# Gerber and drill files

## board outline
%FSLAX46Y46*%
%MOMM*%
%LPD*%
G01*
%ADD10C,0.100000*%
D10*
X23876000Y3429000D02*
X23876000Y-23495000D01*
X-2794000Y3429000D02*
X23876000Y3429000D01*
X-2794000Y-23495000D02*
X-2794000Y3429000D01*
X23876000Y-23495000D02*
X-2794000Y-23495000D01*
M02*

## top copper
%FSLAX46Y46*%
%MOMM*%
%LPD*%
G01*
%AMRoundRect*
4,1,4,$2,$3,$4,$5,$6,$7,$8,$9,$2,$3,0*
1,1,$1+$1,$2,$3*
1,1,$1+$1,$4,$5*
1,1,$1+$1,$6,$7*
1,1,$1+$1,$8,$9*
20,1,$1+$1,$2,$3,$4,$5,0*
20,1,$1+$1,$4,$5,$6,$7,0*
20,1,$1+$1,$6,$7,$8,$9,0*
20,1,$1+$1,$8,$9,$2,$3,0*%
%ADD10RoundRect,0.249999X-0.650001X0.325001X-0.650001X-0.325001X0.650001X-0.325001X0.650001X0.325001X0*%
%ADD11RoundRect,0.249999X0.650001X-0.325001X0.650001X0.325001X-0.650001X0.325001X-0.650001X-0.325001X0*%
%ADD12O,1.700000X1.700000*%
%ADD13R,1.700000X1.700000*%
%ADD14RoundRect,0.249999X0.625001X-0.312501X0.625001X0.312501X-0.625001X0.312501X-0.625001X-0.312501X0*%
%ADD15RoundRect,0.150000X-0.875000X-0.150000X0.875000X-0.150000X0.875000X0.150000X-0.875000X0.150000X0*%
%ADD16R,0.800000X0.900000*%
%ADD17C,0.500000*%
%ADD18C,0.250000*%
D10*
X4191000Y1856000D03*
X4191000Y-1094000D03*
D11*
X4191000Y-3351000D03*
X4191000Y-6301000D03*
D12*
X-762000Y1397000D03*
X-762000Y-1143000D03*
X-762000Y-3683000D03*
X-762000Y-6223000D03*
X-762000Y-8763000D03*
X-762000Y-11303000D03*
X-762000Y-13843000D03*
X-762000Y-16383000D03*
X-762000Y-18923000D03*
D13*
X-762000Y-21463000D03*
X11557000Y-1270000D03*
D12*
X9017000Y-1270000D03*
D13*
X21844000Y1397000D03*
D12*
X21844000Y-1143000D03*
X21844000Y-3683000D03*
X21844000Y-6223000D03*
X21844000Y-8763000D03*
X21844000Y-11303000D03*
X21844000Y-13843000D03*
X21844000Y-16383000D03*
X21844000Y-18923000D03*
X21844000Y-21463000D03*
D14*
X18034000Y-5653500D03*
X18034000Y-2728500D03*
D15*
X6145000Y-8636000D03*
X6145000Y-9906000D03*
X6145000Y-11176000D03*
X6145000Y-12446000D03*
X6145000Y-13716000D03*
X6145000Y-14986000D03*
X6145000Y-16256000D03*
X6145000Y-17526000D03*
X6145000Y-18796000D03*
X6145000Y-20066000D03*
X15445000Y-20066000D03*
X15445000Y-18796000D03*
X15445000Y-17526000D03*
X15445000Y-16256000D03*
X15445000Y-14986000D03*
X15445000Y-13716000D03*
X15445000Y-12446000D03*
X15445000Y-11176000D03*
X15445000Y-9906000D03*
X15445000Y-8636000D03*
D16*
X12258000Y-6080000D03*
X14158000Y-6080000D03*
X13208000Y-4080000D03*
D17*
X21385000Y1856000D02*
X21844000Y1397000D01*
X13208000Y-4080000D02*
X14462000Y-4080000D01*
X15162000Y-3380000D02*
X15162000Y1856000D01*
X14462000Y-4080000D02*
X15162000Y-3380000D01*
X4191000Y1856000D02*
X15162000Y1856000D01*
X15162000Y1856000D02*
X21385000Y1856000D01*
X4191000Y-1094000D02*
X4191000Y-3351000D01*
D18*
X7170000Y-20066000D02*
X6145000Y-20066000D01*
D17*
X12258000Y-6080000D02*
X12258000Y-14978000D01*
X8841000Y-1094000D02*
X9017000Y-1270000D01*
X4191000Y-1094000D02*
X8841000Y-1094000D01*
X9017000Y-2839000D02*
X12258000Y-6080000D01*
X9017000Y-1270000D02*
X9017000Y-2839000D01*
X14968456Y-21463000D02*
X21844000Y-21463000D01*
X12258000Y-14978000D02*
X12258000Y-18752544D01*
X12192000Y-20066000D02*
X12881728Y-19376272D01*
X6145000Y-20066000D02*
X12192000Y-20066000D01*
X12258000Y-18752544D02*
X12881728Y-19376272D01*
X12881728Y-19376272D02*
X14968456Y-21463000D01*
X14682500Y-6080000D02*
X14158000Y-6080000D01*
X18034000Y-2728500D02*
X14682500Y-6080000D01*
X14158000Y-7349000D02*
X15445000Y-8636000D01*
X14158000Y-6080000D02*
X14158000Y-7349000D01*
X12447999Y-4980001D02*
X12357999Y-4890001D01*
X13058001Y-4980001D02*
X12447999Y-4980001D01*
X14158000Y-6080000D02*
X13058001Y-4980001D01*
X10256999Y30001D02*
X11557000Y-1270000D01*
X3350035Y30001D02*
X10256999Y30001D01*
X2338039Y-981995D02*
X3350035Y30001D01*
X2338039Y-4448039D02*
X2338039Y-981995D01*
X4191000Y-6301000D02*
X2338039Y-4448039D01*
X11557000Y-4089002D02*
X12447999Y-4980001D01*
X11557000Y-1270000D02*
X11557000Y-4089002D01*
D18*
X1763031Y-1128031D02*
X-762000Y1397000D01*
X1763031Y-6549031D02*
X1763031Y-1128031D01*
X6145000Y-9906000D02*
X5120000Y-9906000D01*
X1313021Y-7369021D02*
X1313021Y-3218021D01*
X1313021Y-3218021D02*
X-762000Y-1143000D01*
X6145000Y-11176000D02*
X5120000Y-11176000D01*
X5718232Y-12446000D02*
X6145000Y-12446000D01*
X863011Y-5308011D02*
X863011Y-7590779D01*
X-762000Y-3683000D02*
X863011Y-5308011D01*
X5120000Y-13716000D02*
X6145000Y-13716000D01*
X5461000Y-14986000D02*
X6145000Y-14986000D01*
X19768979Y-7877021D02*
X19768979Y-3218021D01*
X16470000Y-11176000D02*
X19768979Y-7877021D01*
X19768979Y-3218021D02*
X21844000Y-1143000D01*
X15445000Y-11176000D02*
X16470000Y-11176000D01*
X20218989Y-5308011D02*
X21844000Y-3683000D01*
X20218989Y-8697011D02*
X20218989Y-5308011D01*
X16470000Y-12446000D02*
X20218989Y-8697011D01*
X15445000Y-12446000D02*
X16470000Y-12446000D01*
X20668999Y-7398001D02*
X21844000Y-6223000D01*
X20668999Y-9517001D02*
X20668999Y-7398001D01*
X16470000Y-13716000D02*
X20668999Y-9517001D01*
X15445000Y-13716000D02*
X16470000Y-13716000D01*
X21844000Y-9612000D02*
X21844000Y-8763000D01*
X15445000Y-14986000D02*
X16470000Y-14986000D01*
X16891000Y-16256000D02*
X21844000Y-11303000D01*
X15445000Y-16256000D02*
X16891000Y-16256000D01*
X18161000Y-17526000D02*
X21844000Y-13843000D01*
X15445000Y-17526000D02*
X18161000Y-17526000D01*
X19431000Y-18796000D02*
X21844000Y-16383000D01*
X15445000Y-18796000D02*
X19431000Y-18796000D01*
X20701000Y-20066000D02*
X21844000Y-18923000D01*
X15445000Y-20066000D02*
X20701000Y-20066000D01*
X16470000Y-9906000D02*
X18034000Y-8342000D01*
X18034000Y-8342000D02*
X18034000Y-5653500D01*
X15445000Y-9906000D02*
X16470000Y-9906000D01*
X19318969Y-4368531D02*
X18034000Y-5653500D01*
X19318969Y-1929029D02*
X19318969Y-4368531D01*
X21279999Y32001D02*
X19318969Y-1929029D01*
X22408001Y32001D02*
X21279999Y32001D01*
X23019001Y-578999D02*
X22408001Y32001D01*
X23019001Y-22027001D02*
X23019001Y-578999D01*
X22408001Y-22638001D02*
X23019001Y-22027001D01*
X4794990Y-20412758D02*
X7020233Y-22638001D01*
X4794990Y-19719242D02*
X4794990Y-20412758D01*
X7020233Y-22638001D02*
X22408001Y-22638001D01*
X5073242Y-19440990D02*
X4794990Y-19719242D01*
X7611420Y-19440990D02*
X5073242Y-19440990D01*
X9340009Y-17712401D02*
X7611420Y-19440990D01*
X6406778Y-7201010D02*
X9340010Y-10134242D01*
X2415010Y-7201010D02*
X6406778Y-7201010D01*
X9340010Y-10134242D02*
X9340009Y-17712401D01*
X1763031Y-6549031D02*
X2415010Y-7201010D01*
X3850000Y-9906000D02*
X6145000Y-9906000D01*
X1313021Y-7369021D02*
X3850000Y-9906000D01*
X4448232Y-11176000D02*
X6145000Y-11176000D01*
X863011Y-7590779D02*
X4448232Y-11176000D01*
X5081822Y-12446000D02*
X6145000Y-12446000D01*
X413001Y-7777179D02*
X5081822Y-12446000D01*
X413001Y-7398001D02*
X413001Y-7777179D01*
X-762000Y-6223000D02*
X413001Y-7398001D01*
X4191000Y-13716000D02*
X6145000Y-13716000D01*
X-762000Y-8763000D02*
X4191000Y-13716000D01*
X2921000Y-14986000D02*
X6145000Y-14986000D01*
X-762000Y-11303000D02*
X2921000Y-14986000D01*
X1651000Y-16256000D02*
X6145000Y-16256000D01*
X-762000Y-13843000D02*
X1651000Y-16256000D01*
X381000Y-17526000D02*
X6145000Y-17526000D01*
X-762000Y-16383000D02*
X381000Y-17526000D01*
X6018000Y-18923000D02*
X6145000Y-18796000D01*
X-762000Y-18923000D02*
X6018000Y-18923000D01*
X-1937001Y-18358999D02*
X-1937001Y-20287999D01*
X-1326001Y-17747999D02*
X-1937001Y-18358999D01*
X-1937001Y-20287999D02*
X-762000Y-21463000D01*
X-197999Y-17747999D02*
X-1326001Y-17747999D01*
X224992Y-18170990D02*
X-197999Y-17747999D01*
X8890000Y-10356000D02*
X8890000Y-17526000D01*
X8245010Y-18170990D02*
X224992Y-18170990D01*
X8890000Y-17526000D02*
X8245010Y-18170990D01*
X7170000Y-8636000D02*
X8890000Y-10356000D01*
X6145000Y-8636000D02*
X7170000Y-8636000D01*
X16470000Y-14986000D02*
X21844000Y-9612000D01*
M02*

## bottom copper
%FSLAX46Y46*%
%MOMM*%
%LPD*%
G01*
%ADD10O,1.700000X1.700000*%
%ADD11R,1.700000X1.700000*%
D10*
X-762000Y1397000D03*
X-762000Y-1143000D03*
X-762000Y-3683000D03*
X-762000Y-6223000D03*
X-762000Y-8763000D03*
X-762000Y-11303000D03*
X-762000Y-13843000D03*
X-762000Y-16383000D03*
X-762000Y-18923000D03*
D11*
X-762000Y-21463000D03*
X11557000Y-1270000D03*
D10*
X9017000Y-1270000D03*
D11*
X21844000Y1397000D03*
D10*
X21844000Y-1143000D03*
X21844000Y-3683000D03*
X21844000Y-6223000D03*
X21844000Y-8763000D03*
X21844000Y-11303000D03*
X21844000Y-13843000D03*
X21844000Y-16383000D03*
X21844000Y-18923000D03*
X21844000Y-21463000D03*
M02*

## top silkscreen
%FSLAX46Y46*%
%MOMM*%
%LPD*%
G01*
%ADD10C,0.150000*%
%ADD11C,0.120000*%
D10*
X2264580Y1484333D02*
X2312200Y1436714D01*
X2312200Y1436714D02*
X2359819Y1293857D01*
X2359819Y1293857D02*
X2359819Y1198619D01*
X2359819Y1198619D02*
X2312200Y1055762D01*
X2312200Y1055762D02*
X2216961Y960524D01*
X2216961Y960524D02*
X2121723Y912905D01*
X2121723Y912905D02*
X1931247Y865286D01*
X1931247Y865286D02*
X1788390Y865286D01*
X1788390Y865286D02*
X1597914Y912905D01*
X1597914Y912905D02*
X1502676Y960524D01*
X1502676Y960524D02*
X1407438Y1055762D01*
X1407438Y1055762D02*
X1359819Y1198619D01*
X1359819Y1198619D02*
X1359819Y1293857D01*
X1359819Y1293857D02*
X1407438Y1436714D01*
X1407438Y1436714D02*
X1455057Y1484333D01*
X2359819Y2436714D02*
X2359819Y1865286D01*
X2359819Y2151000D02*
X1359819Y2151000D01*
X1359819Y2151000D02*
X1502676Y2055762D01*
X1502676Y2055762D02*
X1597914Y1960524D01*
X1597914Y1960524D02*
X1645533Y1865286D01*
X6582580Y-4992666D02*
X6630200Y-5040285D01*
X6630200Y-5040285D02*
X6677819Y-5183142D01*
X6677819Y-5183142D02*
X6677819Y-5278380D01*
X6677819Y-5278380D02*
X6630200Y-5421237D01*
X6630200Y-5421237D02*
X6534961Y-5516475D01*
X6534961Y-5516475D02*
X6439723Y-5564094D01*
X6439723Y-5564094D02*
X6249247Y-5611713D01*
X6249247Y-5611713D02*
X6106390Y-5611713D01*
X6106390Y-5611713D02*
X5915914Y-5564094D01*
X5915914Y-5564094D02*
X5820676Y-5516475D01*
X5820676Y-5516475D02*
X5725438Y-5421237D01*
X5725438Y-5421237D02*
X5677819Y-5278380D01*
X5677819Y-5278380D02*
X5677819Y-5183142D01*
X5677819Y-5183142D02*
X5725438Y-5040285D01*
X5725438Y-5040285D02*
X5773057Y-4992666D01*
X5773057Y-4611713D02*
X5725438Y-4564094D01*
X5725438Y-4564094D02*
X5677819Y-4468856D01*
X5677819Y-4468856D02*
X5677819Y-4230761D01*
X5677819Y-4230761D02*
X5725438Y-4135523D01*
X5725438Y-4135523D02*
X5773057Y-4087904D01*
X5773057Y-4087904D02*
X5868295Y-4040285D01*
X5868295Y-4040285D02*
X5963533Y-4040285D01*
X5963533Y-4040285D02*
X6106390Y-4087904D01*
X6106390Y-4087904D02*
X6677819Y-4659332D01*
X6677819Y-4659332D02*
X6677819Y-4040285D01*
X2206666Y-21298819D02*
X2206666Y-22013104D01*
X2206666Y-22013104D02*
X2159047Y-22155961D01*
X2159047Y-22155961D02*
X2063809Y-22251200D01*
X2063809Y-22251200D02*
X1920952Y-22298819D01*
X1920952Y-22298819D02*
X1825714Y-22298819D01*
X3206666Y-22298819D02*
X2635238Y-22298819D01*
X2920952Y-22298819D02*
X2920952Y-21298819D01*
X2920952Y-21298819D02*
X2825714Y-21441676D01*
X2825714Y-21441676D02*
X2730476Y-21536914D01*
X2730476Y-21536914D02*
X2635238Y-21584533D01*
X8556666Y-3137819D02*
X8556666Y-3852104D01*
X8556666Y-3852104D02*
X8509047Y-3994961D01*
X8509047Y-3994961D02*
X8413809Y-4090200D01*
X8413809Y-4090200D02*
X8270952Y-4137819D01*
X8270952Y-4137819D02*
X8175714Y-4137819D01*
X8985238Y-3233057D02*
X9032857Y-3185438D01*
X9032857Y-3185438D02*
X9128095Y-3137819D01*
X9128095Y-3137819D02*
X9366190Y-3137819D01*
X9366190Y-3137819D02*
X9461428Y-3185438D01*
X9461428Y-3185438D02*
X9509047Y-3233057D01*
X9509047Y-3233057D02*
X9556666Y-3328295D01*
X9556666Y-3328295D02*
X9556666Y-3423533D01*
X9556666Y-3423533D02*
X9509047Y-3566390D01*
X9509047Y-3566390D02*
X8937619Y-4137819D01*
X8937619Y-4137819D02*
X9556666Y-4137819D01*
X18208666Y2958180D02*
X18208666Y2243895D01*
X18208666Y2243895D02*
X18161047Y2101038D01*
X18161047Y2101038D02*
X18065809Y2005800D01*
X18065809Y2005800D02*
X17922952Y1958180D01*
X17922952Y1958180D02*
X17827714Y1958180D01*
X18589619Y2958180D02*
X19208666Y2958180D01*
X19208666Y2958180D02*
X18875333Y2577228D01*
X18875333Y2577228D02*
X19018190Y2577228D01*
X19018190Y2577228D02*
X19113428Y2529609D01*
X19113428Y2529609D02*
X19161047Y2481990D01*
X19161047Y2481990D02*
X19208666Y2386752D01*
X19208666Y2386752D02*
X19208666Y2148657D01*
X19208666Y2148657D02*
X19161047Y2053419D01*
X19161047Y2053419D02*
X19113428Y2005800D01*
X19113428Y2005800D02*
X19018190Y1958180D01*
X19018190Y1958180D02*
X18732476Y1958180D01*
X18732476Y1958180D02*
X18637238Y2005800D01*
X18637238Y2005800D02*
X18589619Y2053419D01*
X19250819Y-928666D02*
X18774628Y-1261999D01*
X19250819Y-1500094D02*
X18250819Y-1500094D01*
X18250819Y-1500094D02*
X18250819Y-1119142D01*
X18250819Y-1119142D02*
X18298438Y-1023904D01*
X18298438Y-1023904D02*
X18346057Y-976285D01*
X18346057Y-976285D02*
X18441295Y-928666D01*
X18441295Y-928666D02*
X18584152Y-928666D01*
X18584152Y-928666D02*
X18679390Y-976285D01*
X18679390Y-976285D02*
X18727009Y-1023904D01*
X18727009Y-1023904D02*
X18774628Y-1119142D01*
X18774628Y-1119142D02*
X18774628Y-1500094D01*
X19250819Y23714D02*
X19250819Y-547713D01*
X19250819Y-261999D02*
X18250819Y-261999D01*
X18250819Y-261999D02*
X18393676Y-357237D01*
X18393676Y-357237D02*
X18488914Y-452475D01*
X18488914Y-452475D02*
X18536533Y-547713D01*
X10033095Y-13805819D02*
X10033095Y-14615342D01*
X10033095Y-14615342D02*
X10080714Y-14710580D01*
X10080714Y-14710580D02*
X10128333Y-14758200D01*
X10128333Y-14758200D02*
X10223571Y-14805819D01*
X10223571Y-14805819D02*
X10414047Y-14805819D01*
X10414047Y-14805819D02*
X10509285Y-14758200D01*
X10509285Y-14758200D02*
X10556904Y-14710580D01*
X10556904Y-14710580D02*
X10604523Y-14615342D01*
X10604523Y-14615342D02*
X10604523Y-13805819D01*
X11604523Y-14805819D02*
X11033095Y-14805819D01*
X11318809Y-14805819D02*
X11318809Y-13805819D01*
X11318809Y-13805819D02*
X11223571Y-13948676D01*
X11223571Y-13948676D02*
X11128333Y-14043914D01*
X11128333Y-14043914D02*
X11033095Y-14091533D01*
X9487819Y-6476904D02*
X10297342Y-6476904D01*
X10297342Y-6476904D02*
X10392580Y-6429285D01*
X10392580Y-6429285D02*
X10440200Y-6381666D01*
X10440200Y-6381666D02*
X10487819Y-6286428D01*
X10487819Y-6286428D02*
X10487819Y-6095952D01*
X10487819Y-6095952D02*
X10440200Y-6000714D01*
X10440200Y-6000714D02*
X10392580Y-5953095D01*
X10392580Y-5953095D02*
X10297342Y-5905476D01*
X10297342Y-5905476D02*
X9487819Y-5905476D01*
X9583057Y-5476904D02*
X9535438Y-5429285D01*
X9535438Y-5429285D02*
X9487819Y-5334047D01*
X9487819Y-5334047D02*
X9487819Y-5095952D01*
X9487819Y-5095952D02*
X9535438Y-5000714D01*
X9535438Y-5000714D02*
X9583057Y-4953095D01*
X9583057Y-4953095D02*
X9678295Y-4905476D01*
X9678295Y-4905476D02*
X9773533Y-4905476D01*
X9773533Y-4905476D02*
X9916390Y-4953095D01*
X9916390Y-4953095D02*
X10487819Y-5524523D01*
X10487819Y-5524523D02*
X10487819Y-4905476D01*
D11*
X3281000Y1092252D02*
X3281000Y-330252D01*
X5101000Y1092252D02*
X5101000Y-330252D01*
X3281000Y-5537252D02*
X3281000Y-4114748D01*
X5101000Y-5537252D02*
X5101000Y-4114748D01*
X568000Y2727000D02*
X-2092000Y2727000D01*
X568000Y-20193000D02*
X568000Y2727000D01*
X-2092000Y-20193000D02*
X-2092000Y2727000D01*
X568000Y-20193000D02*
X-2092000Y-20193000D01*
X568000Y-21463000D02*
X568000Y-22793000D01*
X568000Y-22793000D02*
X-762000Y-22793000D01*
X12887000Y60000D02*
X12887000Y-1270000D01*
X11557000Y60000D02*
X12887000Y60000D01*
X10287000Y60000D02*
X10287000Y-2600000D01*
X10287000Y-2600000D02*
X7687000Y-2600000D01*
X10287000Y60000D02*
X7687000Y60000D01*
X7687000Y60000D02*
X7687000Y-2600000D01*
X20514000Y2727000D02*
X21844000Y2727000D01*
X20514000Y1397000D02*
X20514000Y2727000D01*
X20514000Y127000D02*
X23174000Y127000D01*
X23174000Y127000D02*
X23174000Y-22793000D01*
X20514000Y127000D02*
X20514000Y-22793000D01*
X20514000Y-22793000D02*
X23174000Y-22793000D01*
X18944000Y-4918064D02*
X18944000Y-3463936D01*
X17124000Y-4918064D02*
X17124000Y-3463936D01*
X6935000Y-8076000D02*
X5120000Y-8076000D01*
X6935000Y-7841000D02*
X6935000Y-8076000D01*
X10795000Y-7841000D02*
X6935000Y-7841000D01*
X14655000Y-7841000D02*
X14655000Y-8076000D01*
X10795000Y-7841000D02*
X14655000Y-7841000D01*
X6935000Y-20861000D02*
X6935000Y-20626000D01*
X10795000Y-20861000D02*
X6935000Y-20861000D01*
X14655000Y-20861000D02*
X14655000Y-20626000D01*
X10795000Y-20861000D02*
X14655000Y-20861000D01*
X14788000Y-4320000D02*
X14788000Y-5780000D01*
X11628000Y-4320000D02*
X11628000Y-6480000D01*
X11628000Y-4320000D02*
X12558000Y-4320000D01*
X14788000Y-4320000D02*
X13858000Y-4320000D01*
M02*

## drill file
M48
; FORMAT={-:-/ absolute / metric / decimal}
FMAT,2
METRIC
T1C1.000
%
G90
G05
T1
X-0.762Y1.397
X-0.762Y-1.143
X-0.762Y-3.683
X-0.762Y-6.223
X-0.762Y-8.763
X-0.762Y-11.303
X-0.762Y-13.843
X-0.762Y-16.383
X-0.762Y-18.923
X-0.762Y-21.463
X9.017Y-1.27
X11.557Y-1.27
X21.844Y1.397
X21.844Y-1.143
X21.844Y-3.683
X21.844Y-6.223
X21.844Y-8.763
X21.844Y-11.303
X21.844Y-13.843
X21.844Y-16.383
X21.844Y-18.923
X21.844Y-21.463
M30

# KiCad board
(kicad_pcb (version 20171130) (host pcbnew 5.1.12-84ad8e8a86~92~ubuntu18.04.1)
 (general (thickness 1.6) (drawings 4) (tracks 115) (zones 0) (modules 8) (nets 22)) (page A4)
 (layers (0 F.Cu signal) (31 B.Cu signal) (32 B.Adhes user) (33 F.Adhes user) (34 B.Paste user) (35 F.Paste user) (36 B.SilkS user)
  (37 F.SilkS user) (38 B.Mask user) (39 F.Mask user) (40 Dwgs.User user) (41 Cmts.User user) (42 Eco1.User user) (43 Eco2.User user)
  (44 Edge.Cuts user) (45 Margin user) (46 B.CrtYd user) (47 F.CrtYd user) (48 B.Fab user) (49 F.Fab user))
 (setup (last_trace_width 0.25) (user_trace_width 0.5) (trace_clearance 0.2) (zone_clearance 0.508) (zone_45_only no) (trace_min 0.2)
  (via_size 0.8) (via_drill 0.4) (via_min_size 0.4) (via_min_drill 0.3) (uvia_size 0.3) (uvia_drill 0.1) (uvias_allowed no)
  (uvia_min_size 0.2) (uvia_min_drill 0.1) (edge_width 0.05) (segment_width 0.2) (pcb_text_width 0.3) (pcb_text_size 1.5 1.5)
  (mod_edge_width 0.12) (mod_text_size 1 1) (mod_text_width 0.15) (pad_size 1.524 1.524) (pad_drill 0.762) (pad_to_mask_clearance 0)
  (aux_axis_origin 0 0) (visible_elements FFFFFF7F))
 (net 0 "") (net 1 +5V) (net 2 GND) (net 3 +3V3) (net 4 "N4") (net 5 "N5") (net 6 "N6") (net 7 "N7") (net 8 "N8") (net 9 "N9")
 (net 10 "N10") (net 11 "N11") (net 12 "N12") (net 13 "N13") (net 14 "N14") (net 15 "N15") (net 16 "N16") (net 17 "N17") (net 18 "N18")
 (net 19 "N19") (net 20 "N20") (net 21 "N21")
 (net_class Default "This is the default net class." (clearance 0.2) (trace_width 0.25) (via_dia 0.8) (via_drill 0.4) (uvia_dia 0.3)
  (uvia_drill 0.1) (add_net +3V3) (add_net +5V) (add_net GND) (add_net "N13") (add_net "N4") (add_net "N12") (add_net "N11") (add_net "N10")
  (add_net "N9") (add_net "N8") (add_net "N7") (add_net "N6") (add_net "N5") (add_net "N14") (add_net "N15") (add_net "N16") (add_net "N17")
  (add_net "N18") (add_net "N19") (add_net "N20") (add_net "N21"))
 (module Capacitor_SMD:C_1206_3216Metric (layer F.Cu) (at 4.191 -0.381 270)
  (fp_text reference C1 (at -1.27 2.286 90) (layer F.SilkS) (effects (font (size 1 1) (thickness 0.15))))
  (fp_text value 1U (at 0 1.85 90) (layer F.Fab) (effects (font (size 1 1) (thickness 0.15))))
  (fp_line (start -0.711252 0.91) (end 0.711252 0.91) (layer F.SilkS) (width 0.12))
  (fp_line (start -0.711252 -0.91) (end 0.711252 -0.91) (layer F.SilkS) (width 0.12))
  (pad 1 smd roundrect (at -1.475 0 270) (size 1.15 1.8) (layers F.Cu F.Paste F.Mask) (roundrect_rratio 0.2173904347826087) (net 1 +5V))
  (pad 2 smd roundrect (at 1.475 0 270) (size 1.15 1.8) (layers F.Cu F.Paste F.Mask) (roundrect_rratio 0.2173904347826087) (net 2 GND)))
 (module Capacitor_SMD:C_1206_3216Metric (layer F.Cu) (at 4.191 4.826 90)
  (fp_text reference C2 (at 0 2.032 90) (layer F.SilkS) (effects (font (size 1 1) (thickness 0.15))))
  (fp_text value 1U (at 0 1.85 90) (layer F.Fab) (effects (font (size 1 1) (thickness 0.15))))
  (fp_line (start -0.711252 -0.91) (end 0.711252 -0.91) (layer F.SilkS) (width 0.12))
  (fp_line (start -0.711252 0.91) (end 0.711252 0.91) (layer F.SilkS) (width 0.12))
  (pad 2 smd roundrect (at 1.475 0 90) (size 1.15 1.8) (layers F.Cu F.Paste F.Mask) (roundrect_rratio 0.2173904347826087) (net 2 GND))
  (pad 1 smd roundrect (at -1.475 0 90) (size 1.15 1.8) (layers F.Cu F.Paste F.Mask) (roundrect_rratio 0.2173904347826087) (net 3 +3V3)))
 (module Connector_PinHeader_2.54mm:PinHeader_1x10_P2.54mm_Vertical (layer F.Cu) (at -0.762 21.463 180)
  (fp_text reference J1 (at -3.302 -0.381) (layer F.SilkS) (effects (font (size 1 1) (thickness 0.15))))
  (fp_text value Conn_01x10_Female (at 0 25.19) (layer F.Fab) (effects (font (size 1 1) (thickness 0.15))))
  (fp_line (start -1.33 24.19) (end 1.33 24.19) (layer F.SilkS) (width 0.12))
  (fp_line (start -1.33 1.27) (end -1.33 24.19) (layer F.SilkS) (width 0.12))
  (fp_line (start 1.33 1.27) (end 1.33 24.19) (layer F.SilkS) (width 0.12))
  (fp_line (start -1.33 1.27) (end 1.33 1.27) (layer F.SilkS) (width 0.12))
  (fp_line (start -1.33 0) (end -1.33 -1.33) (layer F.SilkS) (width 0.12))
  (fp_line (start -1.33 -1.33) (end 0 -1.33) (layer F.SilkS) (width 0.12))
  (pad 10 thru_hole oval (at 0 22.86 180) (size 1.7 1.7) (drill 1) (layers *.Cu *.Mask) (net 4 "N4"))
  (pad 9 thru_hole oval (at 0 20.32 180) (size 1.7 1.7) (drill 1) (layers *.Cu *.Mask) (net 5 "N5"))
  (pad 8 thru_hole oval (at 0 17.78 180) (size 1.7 1.7) (drill 1) (layers *.Cu *.Mask) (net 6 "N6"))
  (pad 7 thru_hole oval (at 0 15.24 180) (size 1.7 1.7) (drill 1) (layers *.Cu *.Mask) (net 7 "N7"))
  (pad 6 thru_hole oval (at 0 12.7 180) (size 1.7 1.7) (drill 1) (layers *.Cu *.Mask) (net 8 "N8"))
  (pad 5 thru_hole oval (at 0 10.16 180) (size 1.7 1.7) (drill 1) (layers *.Cu *.Mask) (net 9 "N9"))
  (pad 4 thru_hole oval (at 0 7.62 180) (size 1.7 1.7) (drill 1) (layers *.Cu *.Mask) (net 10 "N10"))
  (pad 3 thru_hole oval (at 0 5.08 180) (size 1.7 1.7) (drill 1) (layers *.Cu *.Mask) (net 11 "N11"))
  (pad 2 thru_hole oval (at 0 2.54 180) (size 1.7 1.7) (drill 1) (layers *.Cu *.Mask) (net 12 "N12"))
  (pad 1 thru_hole rect (at 0 0 180) (size 1.7 1.7) (drill 1) (layers *.Cu *.Mask) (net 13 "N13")))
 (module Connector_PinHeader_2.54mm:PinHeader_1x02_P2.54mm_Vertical (layer F.Cu) (at 11.557 1.27 270)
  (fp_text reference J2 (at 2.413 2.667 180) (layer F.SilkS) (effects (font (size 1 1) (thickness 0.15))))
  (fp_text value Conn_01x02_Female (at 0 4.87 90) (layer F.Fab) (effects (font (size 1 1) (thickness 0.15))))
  (fp_line (start -1.33 -1.33) (end 0 -1.33) (layer F.SilkS) (width 0.12))
  (fp_line (start -1.33 0) (end -1.33 -1.33) (layer F.SilkS) (width 0.12))
  (fp_line (start -1.33 1.27) (end 1.33 1.27) (layer F.SilkS) (width 0.12))
  (fp_line (start 1.33 1.27) (end 1.33 3.87) (layer F.SilkS) (width 0.12))
  (fp_line (start -1.33 1.27) (end -1.33 3.87) (layer F.SilkS) (width 0.12))
  (fp_line (start -1.33 3.87) (end 1.33 3.87) (layer F.SilkS) (width 0.12))
  (pad 1 thru_hole rect (at 0 0 270) (size 1.7 1.7) (drill 1) (layers *.Cu *.Mask) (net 3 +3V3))
  (pad 2 thru_hole oval (at 0 2.54 270) (size 1.7 1.7) (drill 1) (layers *.Cu *.Mask) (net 2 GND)))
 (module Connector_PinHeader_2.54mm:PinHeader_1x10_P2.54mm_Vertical (layer F.Cu) (at 21.844 -1.397)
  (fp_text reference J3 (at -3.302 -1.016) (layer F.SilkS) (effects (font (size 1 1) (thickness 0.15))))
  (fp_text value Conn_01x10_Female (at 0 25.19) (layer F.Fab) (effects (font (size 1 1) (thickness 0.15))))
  (fp_line (start -1.33 -1.33) (end 0 -1.33) (layer F.SilkS) (width 0.12))
  (fp_line (start -1.33 0) (end -1.33 -1.33) (layer F.SilkS) (width 0.12))
  (fp_line (start -1.33 1.27) (end 1.33 1.27) (layer F.SilkS) (width 0.12))
  (fp_line (start 1.33 1.27) (end 1.33 24.19) (layer F.SilkS) (width 0.12))
  (fp_line (start -1.33 1.27) (end -1.33 24.19) (layer F.SilkS) (width 0.12))
  (fp_line (start -1.33 24.19) (end 1.33 24.19) (layer F.SilkS) (width 0.12))
  (pad 1 thru_hole rect (at 0 0) (size 1.7 1.7) (drill 1) (layers *.Cu *.Mask) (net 1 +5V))
  (pad 2 thru_hole oval (at 0 2.54) (size 1.7 1.7) (drill 1) (layers *.Cu *.Mask) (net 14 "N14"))
  (pad 3 thru_hole oval (at 0 5.08) (size 1.7 1.7) (drill 1) (layers *.Cu *.Mask) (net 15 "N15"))
  (pad 4 thru_hole oval (at 0 7.62) (size 1.7 1.7) (drill 1) (layers *.Cu *.Mask) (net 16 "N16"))
  (pad 5 thru_hole oval (at 0 10.16) (size 1.7 1.7) (drill 1) (layers *.Cu *.Mask) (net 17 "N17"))
  (pad 6 thru_hole oval (at 0 12.7) (size 1.7 1.7) (drill 1) (layers *.Cu *.Mask) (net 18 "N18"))
  (pad 7 thru_hole oval (at 0 15.24) (size 1.7 1.7) (drill 1) (layers *.Cu *.Mask) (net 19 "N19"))
  (pad 8 thru_hole oval (at 0 17.78) (size 1.7 1.7) (drill 1) (layers *.Cu *.Mask) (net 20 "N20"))
  (pad 9 thru_hole oval (at 0 20.32) (size 1.7 1.7) (drill 1) (layers *.Cu *.Mask) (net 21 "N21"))
  (pad 10 thru_hole oval (at 0 22.86) (size 1.7 1.7) (drill 1) (layers *.Cu *.Mask) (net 2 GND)))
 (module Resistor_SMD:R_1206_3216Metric (layer F.Cu) (at 18.034 4.191 90)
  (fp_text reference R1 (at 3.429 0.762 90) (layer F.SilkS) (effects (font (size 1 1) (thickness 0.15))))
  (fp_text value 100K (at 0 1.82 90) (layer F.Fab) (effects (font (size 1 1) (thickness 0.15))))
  (fp_line (start -0.727064 0.91) (end 0.727064 0.91) (layer F.SilkS) (width 0.12))
  (fp_line (start -0.727064 -0.91) (end 0.727064 -0.91) (layer F.SilkS) (width 0.12))
  (pad 1 smd roundrect (at -1.4625 0 90) (size 1.125 1.75) (layers F.Cu F.Paste F.Mask) (roundrect_rratio 0.2222213333333333) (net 4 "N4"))
  (pad 2 smd roundrect (at 1.4625 0 90) (size 1.125 1.75) (layers F.Cu F.Paste F.Mask) (roundrect_rratio 0.2222213333333333) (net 3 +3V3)))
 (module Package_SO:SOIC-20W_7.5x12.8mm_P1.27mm (layer F.Cu) (at 10.795 14.351)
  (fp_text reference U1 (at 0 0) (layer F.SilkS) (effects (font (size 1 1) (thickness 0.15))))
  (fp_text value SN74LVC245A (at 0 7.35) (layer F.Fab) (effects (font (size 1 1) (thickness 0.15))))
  (fp_line (start -3.86 -6.275) (end -5.675 -6.275) (layer F.SilkS) (width 0.12))
  (fp_line (start -3.86 -6.51) (end -3.86 -6.275) (layer F.SilkS) (width 0.12))
  (fp_line (start 0 -6.51) (end -3.86 -6.51) (layer F.SilkS) (width 0.12))
  (fp_line (start 3.86 -6.51) (end 3.86 -6.275) (layer F.SilkS) (width 0.12))
  (fp_line (start 0 -6.51) (end 3.86 -6.51) (layer F.SilkS) (width 0.12))
  (fp_line (start -3.86 6.51) (end -3.86 6.275) (layer F.SilkS) (width 0.12))
  (fp_line (start 0 6.51) (end -3.86 6.51) (layer F.SilkS) (width 0.12))
  (fp_line (start 3.86 6.51) (end 3.86 6.275) (layer F.SilkS) (width 0.12))
  (fp_line (start 0 6.51) (end 3.86 6.51) (layer F.SilkS) (width 0.12))
  (pad 1 smd roundrect (at -4.65 -5.715) (size 2.05 0.6) (layers F.Cu F.Paste F.Mask) (roundrect_rratio 0.25) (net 13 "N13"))
  (pad 2 smd roundrect (at -4.65 -4.445) (size 2.05 0.6) (layers F.Cu F.Paste F.Mask) (roundrect_rratio 0.25) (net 5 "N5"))
  (pad 3 smd roundrect (at -4.65 -3.175) (size 2.05 0.6) (layers F.Cu F.Paste F.Mask) (roundrect_rratio 0.25) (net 6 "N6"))
  (pad 4 smd roundrect (at -4.65 -1.905) (size 2.05 0.6) (layers F.Cu F.Paste F.Mask) (roundrect_rratio 0.25) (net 7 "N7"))
  (pad 5 smd roundrect (at -4.65 -0.635) (size 2.05 0.6) (layers F.Cu F.Paste F.Mask) (roundrect_rratio 0.25) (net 8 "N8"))
  (pad 6 smd roundrect (at -4.65 0.635) (size 2.05 0.6) (layers F.Cu F.Paste F.Mask) (roundrect_rratio 0.25) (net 9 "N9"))
  (pad 7 smd roundrect (at -4.65 1.905) (size 2.05 0.6) (layers F.Cu F.Paste F.Mask) (roundrect_rratio 0.25) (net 10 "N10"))
  (pad 8 smd roundrect (at -4.65 3.175) (size 2.05 0.6) (layers F.Cu F.Paste F.Mask) (roundrect_rratio 0.25) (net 11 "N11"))
  (pad 9 smd roundrect (at -4.65 4.445) (size 2.05 0.6) (layers F.Cu F.Paste F.Mask) (roundrect_rratio 0.25) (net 12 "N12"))
  (pad 10 smd roundrect (at -4.65 5.715) (size 2.05 0.6) (layers F.Cu F.Paste F.Mask) (roundrect_rratio 0.25) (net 2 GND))
  (pad 11 smd roundrect (at 4.65 5.715) (size 2.05 0.6) (layers F.Cu F.Paste F.Mask) (roundrect_rratio 0.25) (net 21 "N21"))
  (pad 12 smd roundrect (at 4.65 4.445) (size 2.05 0.6) (layers F.Cu F.Paste F.Mask) (roundrect_rratio 0.25) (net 20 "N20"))
  (pad 13 smd roundrect (at 4.65 3.175) (size 2.05 0.6) (layers F.Cu F.Paste F.Mask) (roundrect_rratio 0.25) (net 19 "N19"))
  (pad 14 smd roundrect (at 4.65 1.905) (size 2.05 0.6) (layers F.Cu F.Paste F.Mask) (roundrect_rratio 0.25) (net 18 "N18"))
  (pad 15 smd roundrect (at 4.65 0.635) (size 2.05 0.6) (layers F.Cu F.Paste F.Mask) (roundrect_rratio 0.25) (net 17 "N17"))
  (pad 16 smd roundrect (at 4.65 -0.635) (size 2.05 0.6) (layers F.Cu F.Paste F.Mask) (roundrect_rratio 0.25) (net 16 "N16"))
  (pad 17 smd roundrect (at 4.65 -1.905) (size 2.05 0.6) (layers F.Cu F.Paste F.Mask) (roundrect_rratio 0.25) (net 15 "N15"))
  (pad 18 smd roundrect (at 4.65 -3.175) (size 2.05 0.6) (layers F.Cu F.Paste F.Mask) (roundrect_rratio 0.25) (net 14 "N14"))
  (pad 19 smd roundrect (at 4.65 -4.445) (size 2.05 0.6) (layers F.Cu F.Paste F.Mask) (roundrect_rratio 0.25) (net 4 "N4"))
  (pad 20 smd roundrect (at 4.65 -5.715) (size 2.05 0.6) (layers F.Cu F.Paste F.Mask) (roundrect_rratio 0.25) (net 3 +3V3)))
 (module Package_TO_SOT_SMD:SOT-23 (layer F.Cu) (at 13.208 5.08 90)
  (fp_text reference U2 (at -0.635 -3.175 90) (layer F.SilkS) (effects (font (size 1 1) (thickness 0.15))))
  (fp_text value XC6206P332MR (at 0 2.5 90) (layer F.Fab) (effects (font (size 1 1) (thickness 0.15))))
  (fp_line (start 0.76 1.58) (end -0.7 1.58) (layer F.SilkS) (width 0.12))
  (fp_line (start 0.76 -1.58) (end -1.4 -1.58) (layer F.SilkS) (width 0.12))
  (fp_line (start 0.76 -1.58) (end 0.76 -0.65) (layer F.SilkS) (width 0.12))
  (fp_line (start 0.76 1.58) (end 0.76 0.65) (layer F.SilkS) (width 0.12))
  (pad 1 smd rect (at -1 -0.95 90) (size 0.9 0.8) (layers F.Cu F.Paste F.Mask) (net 2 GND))
  (pad 2 smd rect (at -1 0.95 90) (size 0.9 0.8) (layers F.Cu F.Paste F.Mask) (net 3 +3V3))
  (pad 3 smd rect (at 1 0 90) (size 0.9 0.8) (layers F.Cu F.Paste F.Mask) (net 1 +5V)))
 (gr_line (start 23.876 -3.429) (end 23.876 23.495) (layer Edge.Cuts) (width 0.1))
 (gr_line (start -2.794 -3.429) (end 23.876 -3.429) (layer Edge.Cuts) (width 0.1))
 (gr_line (start -2.794 23.495) (end -2.794 -3.429) (layer Edge.Cuts) (width 0.1))
 (gr_line (start 23.876 23.495) (end -2.794 23.495) (layer Edge.Cuts) (width 0.1))
 (segment (start 21.385 -1.856) (end 21.844 -1.397) (width 0.5) (layer F.Cu) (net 1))
 (segment (start 13.208 4.08) (end 14.462 4.08) (width 0.5) (layer F.Cu) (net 1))
 (segment (start 15.162 3.38) (end 15.162 -1.856) (width 0.5) (layer F.Cu) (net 1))
 (segment (start 14.462 4.08) (end 15.162 3.38) (width 0.5) (layer F.Cu) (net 1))
 (segment (start 4.191 -1.856) (end 15.162 -1.856) (width 0.5) (layer F.Cu) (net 1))
 (segment (start 15.162 -1.856) (end 21.385 -1.856) (width 0.5) (layer F.Cu) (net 1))
 (segment (start 4.191 1.094) (end 4.191 3.351) (width 0.5) (layer F.Cu) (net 2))
 (segment (start 7.17 20.066) (end 6.145 20.066) (width 0.25) (layer F.Cu) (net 2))
 (segment (start 12.258 6.08) (end 12.258 14.978) (width 0.5) (layer F.Cu) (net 2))
 (segment (start 8.841 1.094) (end 9.017 1.27) (width 0.5) (layer F.Cu) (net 2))
 (segment (start 4.191 1.094) (end 8.841 1.094) (width 0.5) (layer F.Cu) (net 2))
 (segment (start 9.017 2.839) (end 12.258 6.08) (width 0.5) (layer F.Cu) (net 2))
 (segment (start 9.017 1.27) (end 9.017 2.839) (width 0.5) (layer F.Cu) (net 2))
 (segment (start 14.968456 21.463) (end 21.844 21.463) (width 0.5) (layer F.Cu) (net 2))
 (segment (start 12.258 14.978) (end 12.258 18.752544) (width 0.5) (layer F.Cu) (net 2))
 (segment (start 12.192 20.066) (end 12.881728 19.376272) (width 0.5) (layer F.Cu) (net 2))
 (segment (start 6.145 20.066) (end 12.192 20.066) (width 0.5) (layer F.Cu) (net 2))
 (segment (start 12.258 18.752544) (end 12.881728 19.376272) (width 0.5) (layer F.Cu) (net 2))
 (segment (start 12.881728 19.376272) (end 14.968456 21.463) (width 0.5) (layer F.Cu) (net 2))
 (segment (start 14.6825 6.08) (end 14.158 6.08) (width 0.5) (layer F.Cu) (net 3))
 (segment (start 18.034 2.7285) (end 14.6825 6.08) (width 0.5) (layer F.Cu) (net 3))
 (segment (start 14.158 7.349) (end 15.445 8.636) (width 0.5) (layer F.Cu) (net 3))
 (segment (start 14.158 6.08) (end 14.158 7.349) (width 0.5) (layer F.Cu) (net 3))
 (segment (start 12.447999 4.980001) (end 12.357999 4.890001) (width 0.5) (layer F.Cu) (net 3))
 (segment (start 13.058001 4.980001) (end 12.447999 4.980001) (width 0.5) (layer F.Cu) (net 3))
 (segment (start 14.158 6.08) (end 13.058001 4.980001) (width 0.5) (layer F.Cu) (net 3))
 (segment (start 10.256999 -0.030001) (end 11.557 1.27) (width 0.5) (layer F.Cu) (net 3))
 (segment (start 3.350035 -0.030001) (end 10.256999 -0.030001) (width 0.5) (layer F.Cu) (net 3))
 (segment (start 2.338039 0.981995) (end 3.350035 -0.030001) (width 0.5) (layer F.Cu) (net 3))
 (segment (start 2.338039 4.448039) (end 2.338039 0.981995) (width 0.5) (layer F.Cu) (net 3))
 (segment (start 4.191 6.301) (end 2.338039 4.448039) (width 0.5) (layer F.Cu) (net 3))
 (segment (start 11.557 4.089002) (end 12.447999 4.980001) (width 0.5) (layer F.Cu) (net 3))
 (segment (start 11.557 1.27) (end 11.557 4.089002) (width 0.5) (layer F.Cu) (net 3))
 (segment (start 1.763031 1.128031) (end -0.762 -1.397) (width 0.25) (layer F.Cu) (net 4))
 (segment (start 1.763031 6.549031) (end 1.763031 1.128031) (width 0.25) (layer F.Cu) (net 4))
 (segment (start 6.145 9.906) (end 5.12 9.906) (width 0.25) (layer F.Cu) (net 5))
 (segment (start 1.313021 7.369021) (end 1.313021 3.218021) (width 0.25) (layer F.Cu) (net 5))
 (segment (start 1.313021 3.218021) (end -0.762 1.143) (width 0.25) (layer F.Cu) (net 5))
 (segment (start 6.145 11.176) (end 5.12 11.176) (width 0.25) (layer F.Cu) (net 6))
 (segment (start 5.718232 12.446) (end 6.145 12.446) (width 0.25) (layer F.Cu) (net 7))
 (segment (start 0.863011 5.308011) (end 0.863011 7.590779) (width 0.25) (layer F.Cu) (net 6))
 (segment (start -0.762 3.683) (end 0.863011 5.308011) (width 0.25) (layer F.Cu) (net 6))
 (segment (start 5.12 13.716) (end 6.145 13.716) (width 0.25) (layer F.Cu) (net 8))
 (segment (start 5.461 14.986) (end 6.145 14.986) (width 0.25) (layer F.Cu) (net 9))
 (segment (start 19.768979 7.877021) (end 19.768979 3.218021) (width 0.25) (layer F.Cu) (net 14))
 (segment (start 16.47 11.176) (end 19.768979 7.877021) (width 0.25) (layer F.Cu) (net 14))
 (segment (start 19.768979 3.218021) (end 21.844 1.143) (width 0.25) (layer F.Cu) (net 14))
 (segment (start 15.445 11.176) (end 16.47 11.176) (width 0.25) (layer F.Cu) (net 14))
 (segment (start 20.218989 5.308011) (end 21.844 3.683) (width 0.25) (layer F.Cu) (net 15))
 (segment (start 20.218989 8.697011) (end 20.218989 5.308011) (width 0.25) (layer F.Cu) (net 15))
 (segment (start 16.47 12.446) (end 20.218989 8.697011) (width 0.25) (layer F.Cu) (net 15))
 (segment (start 15.445 12.446) (end 16.47 12.446) (width 0.25) (layer F.Cu) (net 15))
 (segment (start 20.668999 7.398001) (end 21.844 6.223) (width 0.25) (layer F.Cu) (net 16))
 (segment (start 20.668999 9.517001) (end 20.668999 7.398001) (width 0.25) (layer F.Cu) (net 16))
 (segment (start 16.47 13.716) (end 20.668999 9.517001) (width 0.25) (layer F.Cu) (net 16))
 (segment (start 15.445 13.716) (end 16.47 13.716) (width 0.25) (layer F.Cu) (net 16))
 (segment (start 21.844 9.612) (end 21.844 8.763) (width 0.25) (layer F.Cu) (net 17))
 (segment (start 15.445 14.986) (end 16.47 14.986) (width 0.25) (layer F.Cu) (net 17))
 (segment (start 16.891 16.256) (end 21.844 11.303) (width 0.25) (layer F.Cu) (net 18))
 (segment (start 15.445 16.256) (end 16.891 16.256) (width 0.25) (layer F.Cu) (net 18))
 (segment (start 18.161 17.526) (end 21.844 13.843) (width 0.25) (layer F.Cu) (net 19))
 (segment (start 15.445 17.526) (end 18.161 17.526) (width 0.25) (layer F.Cu) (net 19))
 (segment (start 19.431 18.796) (end 21.844 16.383) (width 0.25) (layer F.Cu) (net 20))
 (segment (start 15.445 18.796) (end 19.431 18.796) (width 0.25) (layer F.Cu) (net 20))
 (segment (start 20.701 20.066) (end 21.844 18.923) (width 0.25) (layer F.Cu) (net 21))
 (segment (start 15.445 20.066) (end 20.701 20.066) (width 0.25) (layer F.Cu) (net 21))
 (segment (start 16.47 9.906) (end 18.034 8.342) (width 0.25) (layer F.Cu) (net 4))
 (segment (start 18.034 8.342) (end 18.034 5.6535) (width 0.25) (layer F.Cu) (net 4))
 (segment (start 15.445 9.906) (end 16.47 9.906) (width 0.25) (layer F.Cu) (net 4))
 (segment (start 19.318969 4.368531) (end 18.034 5.6535) (width 0.25) (layer F.Cu) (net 4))
 (segment (start 19.318969 1.929029) (end 19.318969 4.368531) (width 0.25) (layer F.Cu) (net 4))
 (segment (start 21.279999 -0.032001) (end 19.318969 1.929029) (width 0.25) (layer F.Cu) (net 4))
 (segment (start 22.408001 -0.032001) (end 21.279999 -0.032001) (width 0.25) (layer F.Cu) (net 4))
 (segment (start 23.019001 0.578999) (end 22.408001 -0.032001) (width 0.25) (layer F.Cu) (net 4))
 (segment (start 23.019001 22.027001) (end 23.019001 0.578999) (width 0.25) (layer F.Cu) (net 4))
 (segment (start 22.408001 22.638001) (end 23.019001 22.027001) (width 0.25) (layer F.Cu) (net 4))
 (segment (start 4.79499 20.412758) (end 7.020233 22.638001) (width 0.25) (layer F.Cu) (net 4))
 (segment (start 4.79499 19.719242) (end 4.79499 20.412758) (width 0.25) (layer F.Cu) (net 4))
 (segment (start 7.020233 22.638001) (end 22.408001 22.638001) (width 0.25) (layer F.Cu) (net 4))
 (segment (start 5.073242 19.44099) (end 4.79499 19.719242) (width 0.25) (layer F.Cu) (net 4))
 (segment (start 7.61142 19.44099) (end 5.073242 19.44099) (width 0.25) (layer F.Cu) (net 4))
 (segment (start 9.340009 17.712401) (end 7.61142 19.44099) (width 0.25) (layer F.Cu) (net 4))
 (segment (start 6.406778 7.20101) (end 9.34001 10.134242) (width 0.25) (layer F.Cu) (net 4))
 (segment (start 2.41501 7.20101) (end 6.406778 7.20101) (width 0.25) (layer F.Cu) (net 4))
 (segment (start 9.34001 10.134242) (end 9.340009 17.712401) (width 0.25) (layer F.Cu) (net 4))
 (segment (start 1.763031 6.549031) (end 2.41501 7.20101) (width 0.25) (layer F.Cu) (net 4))
 (segment (start 3.85 9.906) (end 6.145 9.906) (width 0.25) (layer F.Cu) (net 5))
 (segment (start 1.313021 7.369021) (end 3.85 9.906) (width 0.25) (layer F.Cu) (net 5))
 (segment (start 4.448232 11.176) (end 6.145 11.176) (width 0.25) (layer F.Cu) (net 6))
 (segment (start 0.863011 7.590779) (end 4.448232 11.176) (width 0.25) (layer F.Cu) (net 6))
 (segment (start 5.081822 12.446) (end 6.145 12.446) (width 0.25) (layer F.Cu) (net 7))
 (segment (start 0.413001 7.777179) (end 5.081822 12.446) (width 0.25) (layer F.Cu) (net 7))
 (segment (start 0.413001 7.398001) (end 0.413001 7.777179) (width 0.25) (layer F.Cu) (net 7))
 (segment (start -0.762 6.223) (end 0.413001 7.398001) (width 0.25) (layer F.Cu) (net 7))
 (segment (start 4.191 13.716) (end 6.145 13.716) (width 0.25) (layer F.Cu) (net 8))
 (segment (start -0.762 8.763) (end 4.191 13.716) (width 0.25) (layer F.Cu) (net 8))
 (segment (start 2.921 14.986) (end 6.145 14.986) (width 0.25) (layer F.Cu) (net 9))
 (segment (start -0.762 11.303) (end 2.921 14.986) (width 0.25) (layer F.Cu) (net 9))
 (segment (start 1.651 16.256) (end 6.145 16.256) (width 0.25) (layer F.Cu) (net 10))
 (segment (start -0.762 13.843) (end 1.651 16.256) (width 0.25) (layer F.Cu) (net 10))
 (segment (start 0.381 17.526) (end 6.145 17.526) (width 0.25) (layer F.Cu) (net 11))
 (segment (start -0.762 16.383) (end 0.381 17.526) (width 0.25) (layer F.Cu) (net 11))
 (segment (start 6.018 18.923) (end 6.145 18.796) (width 0.25) (layer F.Cu) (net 12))
 (segment (start -0.762 18.923) (end 6.018 18.923) (width 0.25) (layer F.Cu) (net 12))
 (segment (start -1.937001 18.358999) (end -1.937001 20.287999) (width 0.25) (layer F.Cu) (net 13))
 (segment (start -1.326001 17.747999) (end -1.937001 18.358999) (width 0.25) (layer F.Cu) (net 13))
 (segment (start -1.937001 20.287999) (end -0.762 21.463) (width 0.25) (layer F.Cu) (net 13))
 (segment (start -0.197999 17.747999) (end -1.326001 17.747999) (width 0.25) (layer F.Cu) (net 13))
 (segment (start 0.224992 18.17099) (end -0.197999 17.747999) (width 0.25) (layer F.Cu) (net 13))
 (segment (start 8.89 10.356) (end 8.89 17.526) (width 0.25) (layer F.Cu) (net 13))
 (segment (start 8.24501 18.17099) (end 0.224992 18.17099) (width 0.25) (layer F.Cu) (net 13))
 (segment (start 8.89 17.526) (end 8.24501 18.17099) (width 0.25) (layer F.Cu) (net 13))
 (segment (start 7.17 8.636) (end 8.89 10.356) (width 0.25) (layer F.Cu) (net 13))
 (segment (start 6.145 8.636) (end 7.17 8.636) (width 0.25) (layer F.Cu) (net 13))
 (segment (start 16.47 14.986) (end 21.844 9.612) (width 0.25) (layer F.Cu) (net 17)))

